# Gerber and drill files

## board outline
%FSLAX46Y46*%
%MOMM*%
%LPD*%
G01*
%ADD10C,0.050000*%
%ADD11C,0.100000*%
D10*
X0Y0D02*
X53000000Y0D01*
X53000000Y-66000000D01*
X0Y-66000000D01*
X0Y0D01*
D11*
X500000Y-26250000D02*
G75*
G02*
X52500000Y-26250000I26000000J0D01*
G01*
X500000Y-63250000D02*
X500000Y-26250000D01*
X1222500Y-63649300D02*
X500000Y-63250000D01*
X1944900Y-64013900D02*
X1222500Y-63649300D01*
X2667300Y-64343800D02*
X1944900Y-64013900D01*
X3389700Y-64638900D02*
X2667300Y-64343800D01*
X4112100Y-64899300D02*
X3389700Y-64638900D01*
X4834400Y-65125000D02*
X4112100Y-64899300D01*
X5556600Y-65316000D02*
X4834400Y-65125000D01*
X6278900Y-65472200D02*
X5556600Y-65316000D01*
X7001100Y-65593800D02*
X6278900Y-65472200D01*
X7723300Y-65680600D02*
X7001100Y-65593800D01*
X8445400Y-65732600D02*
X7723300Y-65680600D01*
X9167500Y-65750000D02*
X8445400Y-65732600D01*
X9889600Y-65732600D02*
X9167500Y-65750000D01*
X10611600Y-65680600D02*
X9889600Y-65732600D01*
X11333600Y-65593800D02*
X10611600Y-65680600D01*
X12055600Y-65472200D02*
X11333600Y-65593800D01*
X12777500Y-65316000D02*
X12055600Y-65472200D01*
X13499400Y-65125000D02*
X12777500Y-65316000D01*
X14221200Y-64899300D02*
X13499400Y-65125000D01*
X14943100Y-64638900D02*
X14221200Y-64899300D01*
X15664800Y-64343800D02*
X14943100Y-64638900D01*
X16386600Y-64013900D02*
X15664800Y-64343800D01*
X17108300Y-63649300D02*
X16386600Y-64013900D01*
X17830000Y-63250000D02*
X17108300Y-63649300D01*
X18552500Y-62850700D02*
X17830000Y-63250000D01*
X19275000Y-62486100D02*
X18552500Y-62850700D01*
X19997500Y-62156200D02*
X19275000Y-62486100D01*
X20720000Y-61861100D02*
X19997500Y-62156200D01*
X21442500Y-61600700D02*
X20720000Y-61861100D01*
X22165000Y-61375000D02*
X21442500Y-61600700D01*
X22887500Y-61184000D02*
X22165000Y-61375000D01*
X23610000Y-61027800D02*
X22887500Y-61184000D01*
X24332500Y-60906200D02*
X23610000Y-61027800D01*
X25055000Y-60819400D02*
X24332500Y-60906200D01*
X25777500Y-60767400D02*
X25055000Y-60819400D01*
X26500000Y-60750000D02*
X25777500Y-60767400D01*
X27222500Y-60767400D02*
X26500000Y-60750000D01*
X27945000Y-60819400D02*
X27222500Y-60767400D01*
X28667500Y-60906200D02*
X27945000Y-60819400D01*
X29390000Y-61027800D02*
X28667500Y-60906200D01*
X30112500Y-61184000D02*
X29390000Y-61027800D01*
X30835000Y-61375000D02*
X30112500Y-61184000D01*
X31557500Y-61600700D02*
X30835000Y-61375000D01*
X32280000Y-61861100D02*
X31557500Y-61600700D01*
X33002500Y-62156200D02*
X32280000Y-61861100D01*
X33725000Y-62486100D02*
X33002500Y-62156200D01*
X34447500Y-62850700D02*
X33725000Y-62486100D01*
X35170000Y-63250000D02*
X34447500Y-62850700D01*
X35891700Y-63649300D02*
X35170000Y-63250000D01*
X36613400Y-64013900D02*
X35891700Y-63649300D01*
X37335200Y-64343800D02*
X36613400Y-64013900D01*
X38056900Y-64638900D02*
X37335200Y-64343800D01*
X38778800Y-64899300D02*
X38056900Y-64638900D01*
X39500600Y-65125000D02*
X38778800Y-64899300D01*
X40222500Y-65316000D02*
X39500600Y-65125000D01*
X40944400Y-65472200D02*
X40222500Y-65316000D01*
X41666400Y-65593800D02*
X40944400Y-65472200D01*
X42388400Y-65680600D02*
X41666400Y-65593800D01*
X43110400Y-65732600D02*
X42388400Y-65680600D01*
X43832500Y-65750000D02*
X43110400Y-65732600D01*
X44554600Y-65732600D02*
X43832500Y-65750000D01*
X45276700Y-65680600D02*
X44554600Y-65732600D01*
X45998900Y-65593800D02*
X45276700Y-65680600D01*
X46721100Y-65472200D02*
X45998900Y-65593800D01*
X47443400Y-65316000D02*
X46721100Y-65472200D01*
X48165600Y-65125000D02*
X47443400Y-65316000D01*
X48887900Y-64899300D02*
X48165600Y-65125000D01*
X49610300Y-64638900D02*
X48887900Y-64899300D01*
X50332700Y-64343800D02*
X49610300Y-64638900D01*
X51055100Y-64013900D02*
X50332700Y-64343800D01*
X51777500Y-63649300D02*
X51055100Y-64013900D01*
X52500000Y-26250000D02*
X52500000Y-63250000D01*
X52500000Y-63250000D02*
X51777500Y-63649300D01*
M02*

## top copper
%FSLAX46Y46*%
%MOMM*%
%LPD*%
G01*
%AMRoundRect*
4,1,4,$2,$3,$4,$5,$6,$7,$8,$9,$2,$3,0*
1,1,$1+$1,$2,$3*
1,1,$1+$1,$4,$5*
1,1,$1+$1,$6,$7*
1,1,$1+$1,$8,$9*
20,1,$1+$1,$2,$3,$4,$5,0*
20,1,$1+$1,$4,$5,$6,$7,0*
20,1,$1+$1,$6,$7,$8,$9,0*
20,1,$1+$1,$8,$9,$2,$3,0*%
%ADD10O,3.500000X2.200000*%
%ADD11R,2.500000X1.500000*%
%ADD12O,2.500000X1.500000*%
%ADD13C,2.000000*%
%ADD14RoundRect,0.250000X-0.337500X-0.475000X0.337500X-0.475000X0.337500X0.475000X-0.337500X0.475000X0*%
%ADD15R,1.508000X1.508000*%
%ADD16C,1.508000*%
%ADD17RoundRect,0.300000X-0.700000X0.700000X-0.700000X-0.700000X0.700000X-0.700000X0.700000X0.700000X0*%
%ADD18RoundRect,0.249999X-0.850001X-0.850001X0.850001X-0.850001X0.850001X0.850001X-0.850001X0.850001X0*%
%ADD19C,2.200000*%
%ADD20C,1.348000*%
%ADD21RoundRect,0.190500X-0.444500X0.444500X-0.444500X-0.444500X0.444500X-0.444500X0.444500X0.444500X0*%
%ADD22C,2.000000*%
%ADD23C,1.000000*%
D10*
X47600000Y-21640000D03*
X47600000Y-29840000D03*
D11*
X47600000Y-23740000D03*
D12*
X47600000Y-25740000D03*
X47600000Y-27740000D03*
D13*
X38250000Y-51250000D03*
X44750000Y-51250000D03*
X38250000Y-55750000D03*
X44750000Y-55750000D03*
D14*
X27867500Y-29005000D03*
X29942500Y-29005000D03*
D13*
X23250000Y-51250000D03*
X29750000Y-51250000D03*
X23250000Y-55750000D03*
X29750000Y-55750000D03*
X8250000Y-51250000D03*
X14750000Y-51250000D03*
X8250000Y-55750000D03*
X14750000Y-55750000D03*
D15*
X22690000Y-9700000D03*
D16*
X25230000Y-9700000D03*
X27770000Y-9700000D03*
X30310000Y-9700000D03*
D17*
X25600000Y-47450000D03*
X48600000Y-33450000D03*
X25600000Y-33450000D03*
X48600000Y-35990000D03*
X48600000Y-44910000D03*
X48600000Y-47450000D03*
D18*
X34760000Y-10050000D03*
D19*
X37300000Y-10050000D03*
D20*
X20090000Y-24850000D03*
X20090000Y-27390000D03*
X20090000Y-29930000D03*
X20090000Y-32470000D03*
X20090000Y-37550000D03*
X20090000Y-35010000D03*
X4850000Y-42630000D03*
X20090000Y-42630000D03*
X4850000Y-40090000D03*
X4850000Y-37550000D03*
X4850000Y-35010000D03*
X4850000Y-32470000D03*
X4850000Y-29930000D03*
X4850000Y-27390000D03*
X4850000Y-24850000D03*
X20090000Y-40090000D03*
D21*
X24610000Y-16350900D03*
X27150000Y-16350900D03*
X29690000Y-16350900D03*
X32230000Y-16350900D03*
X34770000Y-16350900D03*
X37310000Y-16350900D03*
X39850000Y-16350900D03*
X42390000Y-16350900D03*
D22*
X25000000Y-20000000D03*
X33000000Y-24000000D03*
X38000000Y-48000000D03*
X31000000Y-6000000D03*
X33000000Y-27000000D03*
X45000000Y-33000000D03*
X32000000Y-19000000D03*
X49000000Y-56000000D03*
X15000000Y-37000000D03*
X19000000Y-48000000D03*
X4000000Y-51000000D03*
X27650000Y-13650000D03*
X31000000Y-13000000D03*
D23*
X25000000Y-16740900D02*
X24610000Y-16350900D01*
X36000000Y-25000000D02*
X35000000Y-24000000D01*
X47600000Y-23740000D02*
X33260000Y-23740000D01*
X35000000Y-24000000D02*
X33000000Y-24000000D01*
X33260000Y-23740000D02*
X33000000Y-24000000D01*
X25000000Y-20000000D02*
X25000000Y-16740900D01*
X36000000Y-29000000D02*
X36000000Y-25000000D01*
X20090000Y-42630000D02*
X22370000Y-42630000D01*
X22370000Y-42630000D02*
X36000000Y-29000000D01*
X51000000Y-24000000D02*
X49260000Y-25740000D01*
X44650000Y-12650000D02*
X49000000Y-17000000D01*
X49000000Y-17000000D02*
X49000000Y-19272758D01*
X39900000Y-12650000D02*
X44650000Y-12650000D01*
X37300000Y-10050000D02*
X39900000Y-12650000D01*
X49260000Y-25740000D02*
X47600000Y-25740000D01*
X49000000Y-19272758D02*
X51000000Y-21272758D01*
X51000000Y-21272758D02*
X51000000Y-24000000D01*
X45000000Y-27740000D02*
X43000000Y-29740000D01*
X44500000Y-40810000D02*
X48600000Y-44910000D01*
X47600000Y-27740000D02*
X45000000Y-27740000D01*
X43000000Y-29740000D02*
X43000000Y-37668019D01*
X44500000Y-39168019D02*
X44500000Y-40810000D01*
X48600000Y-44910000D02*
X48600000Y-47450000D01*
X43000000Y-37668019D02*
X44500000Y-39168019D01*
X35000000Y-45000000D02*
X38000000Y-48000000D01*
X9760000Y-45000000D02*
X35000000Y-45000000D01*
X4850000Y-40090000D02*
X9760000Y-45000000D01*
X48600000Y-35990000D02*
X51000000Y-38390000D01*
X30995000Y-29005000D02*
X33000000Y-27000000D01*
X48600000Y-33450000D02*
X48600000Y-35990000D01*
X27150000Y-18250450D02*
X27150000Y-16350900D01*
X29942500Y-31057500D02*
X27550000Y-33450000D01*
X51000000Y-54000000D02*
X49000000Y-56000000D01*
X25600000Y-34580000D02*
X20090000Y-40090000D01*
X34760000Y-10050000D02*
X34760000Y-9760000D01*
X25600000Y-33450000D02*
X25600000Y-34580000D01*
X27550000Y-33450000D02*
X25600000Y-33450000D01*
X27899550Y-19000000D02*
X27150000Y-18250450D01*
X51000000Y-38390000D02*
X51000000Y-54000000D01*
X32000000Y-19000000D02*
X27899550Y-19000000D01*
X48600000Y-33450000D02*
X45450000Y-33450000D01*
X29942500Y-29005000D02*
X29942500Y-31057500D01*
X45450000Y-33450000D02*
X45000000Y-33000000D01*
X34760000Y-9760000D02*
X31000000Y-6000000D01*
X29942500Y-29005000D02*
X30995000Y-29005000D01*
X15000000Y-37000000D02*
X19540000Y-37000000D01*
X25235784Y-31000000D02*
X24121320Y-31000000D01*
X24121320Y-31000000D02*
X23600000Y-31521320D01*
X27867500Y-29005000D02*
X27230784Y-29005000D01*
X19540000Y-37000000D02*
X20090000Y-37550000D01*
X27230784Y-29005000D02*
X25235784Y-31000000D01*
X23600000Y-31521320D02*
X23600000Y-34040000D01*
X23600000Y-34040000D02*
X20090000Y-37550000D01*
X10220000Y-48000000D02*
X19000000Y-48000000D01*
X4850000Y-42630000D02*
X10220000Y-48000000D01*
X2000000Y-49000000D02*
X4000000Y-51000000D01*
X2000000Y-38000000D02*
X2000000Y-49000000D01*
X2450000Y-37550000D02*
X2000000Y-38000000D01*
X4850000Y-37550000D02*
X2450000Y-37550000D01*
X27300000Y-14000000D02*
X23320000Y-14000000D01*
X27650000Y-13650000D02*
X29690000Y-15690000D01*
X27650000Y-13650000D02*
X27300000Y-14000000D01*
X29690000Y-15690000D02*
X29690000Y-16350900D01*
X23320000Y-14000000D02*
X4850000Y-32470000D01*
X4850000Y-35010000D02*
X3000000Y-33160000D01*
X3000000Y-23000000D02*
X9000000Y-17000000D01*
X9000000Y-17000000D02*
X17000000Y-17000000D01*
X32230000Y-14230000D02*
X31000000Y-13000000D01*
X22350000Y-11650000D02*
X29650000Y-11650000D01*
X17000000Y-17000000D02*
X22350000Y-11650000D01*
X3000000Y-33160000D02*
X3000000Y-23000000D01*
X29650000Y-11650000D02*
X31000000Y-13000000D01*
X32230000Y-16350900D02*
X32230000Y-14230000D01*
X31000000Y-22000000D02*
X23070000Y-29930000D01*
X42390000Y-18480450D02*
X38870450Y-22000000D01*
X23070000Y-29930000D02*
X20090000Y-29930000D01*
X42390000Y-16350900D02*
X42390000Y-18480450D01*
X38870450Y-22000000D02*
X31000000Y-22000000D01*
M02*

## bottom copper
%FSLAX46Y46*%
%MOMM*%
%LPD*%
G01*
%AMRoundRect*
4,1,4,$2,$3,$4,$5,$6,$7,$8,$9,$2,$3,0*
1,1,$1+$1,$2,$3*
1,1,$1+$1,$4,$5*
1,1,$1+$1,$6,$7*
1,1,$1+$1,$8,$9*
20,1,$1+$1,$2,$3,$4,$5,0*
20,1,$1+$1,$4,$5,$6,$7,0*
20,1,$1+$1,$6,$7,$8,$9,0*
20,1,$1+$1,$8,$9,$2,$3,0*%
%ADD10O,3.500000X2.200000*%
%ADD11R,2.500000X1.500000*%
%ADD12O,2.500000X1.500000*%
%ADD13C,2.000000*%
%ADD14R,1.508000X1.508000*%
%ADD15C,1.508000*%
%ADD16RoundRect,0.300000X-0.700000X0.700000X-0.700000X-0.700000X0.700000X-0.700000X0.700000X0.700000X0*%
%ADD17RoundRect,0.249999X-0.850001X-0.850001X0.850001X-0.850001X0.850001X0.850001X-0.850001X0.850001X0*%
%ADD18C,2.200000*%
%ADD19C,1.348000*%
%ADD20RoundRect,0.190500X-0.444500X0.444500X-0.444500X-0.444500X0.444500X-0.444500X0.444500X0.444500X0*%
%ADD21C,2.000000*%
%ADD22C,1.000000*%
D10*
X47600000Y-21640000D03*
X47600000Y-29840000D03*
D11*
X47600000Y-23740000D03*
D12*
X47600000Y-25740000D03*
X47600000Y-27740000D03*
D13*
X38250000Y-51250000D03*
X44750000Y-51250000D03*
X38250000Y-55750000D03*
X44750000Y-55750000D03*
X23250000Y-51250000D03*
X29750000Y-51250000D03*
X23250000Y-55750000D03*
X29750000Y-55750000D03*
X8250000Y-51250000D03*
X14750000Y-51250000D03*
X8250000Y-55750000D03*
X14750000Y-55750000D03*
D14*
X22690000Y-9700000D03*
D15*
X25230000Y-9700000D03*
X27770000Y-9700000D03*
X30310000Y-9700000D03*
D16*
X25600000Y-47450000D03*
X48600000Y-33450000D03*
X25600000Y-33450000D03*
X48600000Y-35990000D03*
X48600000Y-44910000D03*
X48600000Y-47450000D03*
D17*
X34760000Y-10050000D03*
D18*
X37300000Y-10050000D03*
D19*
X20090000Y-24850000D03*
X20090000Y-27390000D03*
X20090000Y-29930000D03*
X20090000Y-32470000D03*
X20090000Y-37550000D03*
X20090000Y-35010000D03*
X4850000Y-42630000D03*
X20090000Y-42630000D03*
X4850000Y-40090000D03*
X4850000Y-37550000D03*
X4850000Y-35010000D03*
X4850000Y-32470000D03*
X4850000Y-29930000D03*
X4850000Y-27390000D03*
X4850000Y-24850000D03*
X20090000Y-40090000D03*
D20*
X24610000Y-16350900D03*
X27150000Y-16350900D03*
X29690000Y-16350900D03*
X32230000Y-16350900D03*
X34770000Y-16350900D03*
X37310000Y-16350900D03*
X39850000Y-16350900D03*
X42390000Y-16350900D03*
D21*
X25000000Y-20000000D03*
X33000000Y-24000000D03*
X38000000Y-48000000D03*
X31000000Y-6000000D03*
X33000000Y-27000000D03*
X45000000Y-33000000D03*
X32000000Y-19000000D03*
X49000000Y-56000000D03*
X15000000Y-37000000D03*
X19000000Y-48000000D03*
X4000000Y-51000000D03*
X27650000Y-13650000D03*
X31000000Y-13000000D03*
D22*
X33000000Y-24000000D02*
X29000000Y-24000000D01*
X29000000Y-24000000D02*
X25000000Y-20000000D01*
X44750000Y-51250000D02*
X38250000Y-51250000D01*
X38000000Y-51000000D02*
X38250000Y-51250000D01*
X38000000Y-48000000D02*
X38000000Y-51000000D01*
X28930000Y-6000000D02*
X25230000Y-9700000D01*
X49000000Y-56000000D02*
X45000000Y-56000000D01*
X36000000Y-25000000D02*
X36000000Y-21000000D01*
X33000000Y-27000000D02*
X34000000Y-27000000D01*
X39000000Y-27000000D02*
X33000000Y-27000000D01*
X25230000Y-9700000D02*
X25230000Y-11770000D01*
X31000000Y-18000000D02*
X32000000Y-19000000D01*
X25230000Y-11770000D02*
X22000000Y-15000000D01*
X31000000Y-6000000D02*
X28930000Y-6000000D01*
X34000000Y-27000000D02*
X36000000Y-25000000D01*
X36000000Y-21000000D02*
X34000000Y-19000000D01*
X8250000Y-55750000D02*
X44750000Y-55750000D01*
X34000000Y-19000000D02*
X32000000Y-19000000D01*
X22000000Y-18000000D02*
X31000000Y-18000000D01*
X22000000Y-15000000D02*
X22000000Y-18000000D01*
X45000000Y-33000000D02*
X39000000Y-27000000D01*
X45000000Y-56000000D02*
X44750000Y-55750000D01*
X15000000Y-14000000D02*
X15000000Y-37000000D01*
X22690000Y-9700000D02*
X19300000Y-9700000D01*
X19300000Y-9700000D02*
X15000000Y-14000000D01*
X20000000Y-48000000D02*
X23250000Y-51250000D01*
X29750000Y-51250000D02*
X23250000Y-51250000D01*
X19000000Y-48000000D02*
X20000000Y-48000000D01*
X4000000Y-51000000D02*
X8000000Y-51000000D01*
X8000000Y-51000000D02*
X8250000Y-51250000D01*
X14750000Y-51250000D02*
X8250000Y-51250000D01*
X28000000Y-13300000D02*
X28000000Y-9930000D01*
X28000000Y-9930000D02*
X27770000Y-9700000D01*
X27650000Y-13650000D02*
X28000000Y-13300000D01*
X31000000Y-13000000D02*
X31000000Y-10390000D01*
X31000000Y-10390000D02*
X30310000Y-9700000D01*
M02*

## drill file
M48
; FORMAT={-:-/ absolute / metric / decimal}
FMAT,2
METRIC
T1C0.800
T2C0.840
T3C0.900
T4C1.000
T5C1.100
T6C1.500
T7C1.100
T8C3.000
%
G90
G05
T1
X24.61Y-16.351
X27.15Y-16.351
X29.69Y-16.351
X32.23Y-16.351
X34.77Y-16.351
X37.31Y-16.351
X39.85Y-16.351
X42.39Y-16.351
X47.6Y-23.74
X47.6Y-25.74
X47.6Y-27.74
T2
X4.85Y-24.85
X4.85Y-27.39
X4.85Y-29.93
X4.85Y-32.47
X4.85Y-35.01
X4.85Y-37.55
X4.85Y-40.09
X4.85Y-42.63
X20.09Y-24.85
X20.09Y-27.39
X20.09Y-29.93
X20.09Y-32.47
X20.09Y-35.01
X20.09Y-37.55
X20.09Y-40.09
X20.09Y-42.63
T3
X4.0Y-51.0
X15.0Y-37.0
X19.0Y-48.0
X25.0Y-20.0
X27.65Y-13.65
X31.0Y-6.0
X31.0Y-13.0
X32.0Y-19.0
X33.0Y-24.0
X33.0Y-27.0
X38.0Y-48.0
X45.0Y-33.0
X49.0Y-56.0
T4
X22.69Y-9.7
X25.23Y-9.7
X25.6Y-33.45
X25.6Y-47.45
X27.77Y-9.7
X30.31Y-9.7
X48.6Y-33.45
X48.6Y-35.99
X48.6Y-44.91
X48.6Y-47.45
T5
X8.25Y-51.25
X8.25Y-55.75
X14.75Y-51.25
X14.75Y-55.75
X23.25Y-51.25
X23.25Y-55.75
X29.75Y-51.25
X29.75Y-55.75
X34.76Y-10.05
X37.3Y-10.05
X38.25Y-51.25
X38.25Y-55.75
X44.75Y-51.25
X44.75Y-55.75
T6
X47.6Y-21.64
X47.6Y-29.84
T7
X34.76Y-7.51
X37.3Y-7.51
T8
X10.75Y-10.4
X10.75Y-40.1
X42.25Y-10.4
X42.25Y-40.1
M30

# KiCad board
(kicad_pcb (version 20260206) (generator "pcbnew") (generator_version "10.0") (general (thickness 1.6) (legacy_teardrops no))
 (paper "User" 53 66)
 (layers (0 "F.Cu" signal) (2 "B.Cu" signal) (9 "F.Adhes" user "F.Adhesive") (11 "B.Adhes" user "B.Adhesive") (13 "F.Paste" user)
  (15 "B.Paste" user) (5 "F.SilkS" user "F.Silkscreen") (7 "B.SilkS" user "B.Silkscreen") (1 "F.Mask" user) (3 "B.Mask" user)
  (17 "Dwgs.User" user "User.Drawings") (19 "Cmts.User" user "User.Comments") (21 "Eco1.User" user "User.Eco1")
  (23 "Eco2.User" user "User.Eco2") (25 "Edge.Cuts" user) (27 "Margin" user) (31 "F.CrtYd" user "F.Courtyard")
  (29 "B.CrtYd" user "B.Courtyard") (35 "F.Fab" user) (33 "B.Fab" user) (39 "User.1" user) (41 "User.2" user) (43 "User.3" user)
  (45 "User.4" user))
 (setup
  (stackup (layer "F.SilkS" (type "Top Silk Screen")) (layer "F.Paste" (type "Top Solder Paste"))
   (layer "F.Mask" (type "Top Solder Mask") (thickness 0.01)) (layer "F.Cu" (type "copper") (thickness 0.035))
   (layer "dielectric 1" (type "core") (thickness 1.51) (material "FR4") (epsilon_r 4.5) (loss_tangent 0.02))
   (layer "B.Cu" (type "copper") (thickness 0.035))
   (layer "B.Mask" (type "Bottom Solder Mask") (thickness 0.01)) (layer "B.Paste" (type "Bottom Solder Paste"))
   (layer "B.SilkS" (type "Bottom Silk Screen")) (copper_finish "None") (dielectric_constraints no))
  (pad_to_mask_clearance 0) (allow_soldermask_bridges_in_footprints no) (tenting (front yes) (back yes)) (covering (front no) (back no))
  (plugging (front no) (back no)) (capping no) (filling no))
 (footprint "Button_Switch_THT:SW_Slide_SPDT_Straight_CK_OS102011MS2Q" (layer "F.Cu") (at 47.6 23.74 -90)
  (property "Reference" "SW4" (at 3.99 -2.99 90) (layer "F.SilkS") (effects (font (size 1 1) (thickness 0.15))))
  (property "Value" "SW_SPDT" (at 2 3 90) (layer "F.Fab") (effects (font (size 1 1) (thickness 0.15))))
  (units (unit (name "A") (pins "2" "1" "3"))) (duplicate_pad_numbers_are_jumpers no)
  (pad "" thru_hole oval (at -2.1 0 270) (size 2.2 3.5) (drill 1.5) (layers "*.Cu" "*.Mask") (remove_unused_layers no))
  (pad "" thru_hole oval (at 6.1 0 270) (size 2.2 3.5) (drill 1.5) (layers "*.Cu" "*.Mask") (remove_unused_layers no))
  (pad "1" thru_hole rect (at 0 0 270) (size 1.5 2.5) (drill 0.8) (layers "*.Cu" "*.Mask") (remove_unused_layers no) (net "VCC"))
  (pad "2" thru_hole oval (at 2 0 270) (size 1.5 2.5) (drill 0.8) (layers "*.Cu" "*.Mask") (remove_unused_layers no) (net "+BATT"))
  (pad "3" thru_hole oval (at 4 0 270) (size 1.5 2.5) (drill 0.8) (layers "*.Cu" "*.Mask") (remove_unused_layers no) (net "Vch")))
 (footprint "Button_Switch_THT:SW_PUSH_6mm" (layer "F.Cu") (at 38.25 51.25)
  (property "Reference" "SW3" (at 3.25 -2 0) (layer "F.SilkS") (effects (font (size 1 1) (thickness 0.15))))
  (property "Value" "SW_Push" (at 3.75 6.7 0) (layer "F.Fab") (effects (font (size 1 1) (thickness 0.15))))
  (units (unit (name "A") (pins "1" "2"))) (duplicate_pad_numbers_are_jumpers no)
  (pad "1" thru_hole circle (at 0 0 90) (size 2 2) (drill 1.1) (layers "*.Cu" "*.Mask") (remove_unused_layers no) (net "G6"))
  (pad "1" thru_hole circle (at 6.5 0 90) (size 2 2) (drill 1.1) (layers "*.Cu" "*.Mask") (remove_unused_layers no) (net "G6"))
  (pad "2" thru_hole circle (at 0 4.5 90) (size 2 2) (drill 1.1) (layers "*.Cu" "*.Mask") (remove_unused_layers no) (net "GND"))
  (pad "2" thru_hole circle (at 6.5 4.5 90) (size 2 2) (drill 1.1) (layers "*.Cu" "*.Mask") (remove_unused_layers no) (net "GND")))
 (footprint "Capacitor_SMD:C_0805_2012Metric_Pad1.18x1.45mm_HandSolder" (layer "F.Cu") (at 28.905 29.005)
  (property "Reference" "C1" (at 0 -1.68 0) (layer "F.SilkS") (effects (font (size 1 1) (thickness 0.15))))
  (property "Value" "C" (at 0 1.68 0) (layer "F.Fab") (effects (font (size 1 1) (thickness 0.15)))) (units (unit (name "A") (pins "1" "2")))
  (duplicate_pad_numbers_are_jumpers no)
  (pad "1" smd roundrect (at -1.0375 0) (size 1.175 1.45) (layers "F.Cu" "F.Mask" "F.Paste") (roundrect_rratio 0.212766) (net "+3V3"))
  (pad "2" smd roundrect (at 1.0375 0) (size 1.175 1.45) (layers "F.Cu" "F.Mask" "F.Paste") (roundrect_rratio 0.212766) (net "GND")))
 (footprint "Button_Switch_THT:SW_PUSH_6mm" (layer "F.Cu") (at 23.25 51.25)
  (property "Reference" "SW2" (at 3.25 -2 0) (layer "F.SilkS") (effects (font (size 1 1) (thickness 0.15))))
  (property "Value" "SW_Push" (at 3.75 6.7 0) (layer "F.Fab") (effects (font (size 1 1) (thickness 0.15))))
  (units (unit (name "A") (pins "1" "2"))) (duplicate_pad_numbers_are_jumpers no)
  (pad "1" thru_hole circle (at 0 0 90) (size 2 2) (drill 1.1) (layers "*.Cu" "*.Mask") (remove_unused_layers no) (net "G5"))
  (pad "1" thru_hole circle (at 6.5 0 90) (size 2 2) (drill 1.1) (layers "*.Cu" "*.Mask") (remove_unused_layers no) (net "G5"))
  (pad "2" thru_hole circle (at 0 4.5 90) (size 2 2) (drill 1.1) (layers "*.Cu" "*.Mask") (remove_unused_layers no) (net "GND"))
  (pad "2" thru_hole circle (at 6.5 4.5 90) (size 2 2) (drill 1.1) (layers "*.Cu" "*.Mask") (remove_unused_layers no) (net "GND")))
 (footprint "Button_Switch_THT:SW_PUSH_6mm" (layer "F.Cu") (at 8.25 51.25)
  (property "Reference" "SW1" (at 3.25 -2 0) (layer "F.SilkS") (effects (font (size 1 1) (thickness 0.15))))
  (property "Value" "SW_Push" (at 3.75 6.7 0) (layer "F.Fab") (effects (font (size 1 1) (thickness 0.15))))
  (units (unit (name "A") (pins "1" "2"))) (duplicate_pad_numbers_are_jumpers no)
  (pad "1" thru_hole circle (at 0 0 90) (size 2 2) (drill 1.1) (layers "*.Cu" "*.Mask") (remove_unused_layers no) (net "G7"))
  (pad "1" thru_hole circle (at 6.5 0 90) (size 2 2) (drill 1.1) (layers "*.Cu" "*.Mask") (remove_unused_layers no) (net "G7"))
  (pad "2" thru_hole circle (at 0 4.5 90) (size 2 2) (drill 1.1) (layers "*.Cu" "*.Mask") (remove_unused_layers no) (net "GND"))
  (pad "2" thru_hole circle (at 6.5 4.5 90) (size 2 2) (drill 1.1) (layers "*.Cu" "*.Mask") (remove_unused_layers no) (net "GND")))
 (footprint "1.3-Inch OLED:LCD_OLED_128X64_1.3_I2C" (layer "F.Cu") (at 26.5 25.25)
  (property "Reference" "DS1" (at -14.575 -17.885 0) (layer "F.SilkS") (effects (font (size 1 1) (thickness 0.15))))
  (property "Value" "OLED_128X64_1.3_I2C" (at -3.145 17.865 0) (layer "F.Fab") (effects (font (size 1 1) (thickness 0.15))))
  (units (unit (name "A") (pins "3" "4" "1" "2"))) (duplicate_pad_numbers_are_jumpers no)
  (pad "" np_thru_hole circle (at -15.75 -14.85) (size 3 3) (drill 3) (layers "*.Cu" "*.Mask"))
  (pad "" np_thru_hole circle (at -15.75 14.85) (size 3 3) (drill 3) (layers "*.Cu" "*.Mask"))
  (pad "" np_thru_hole circle (at 15.75 -14.85) (size 3 3) (drill 3) (layers "*.Cu" "*.Mask"))
  (pad "" np_thru_hole circle (at 15.75 14.85) (size 3 3) (drill 3) (layers "*.Cu" "*.Mask"))
  (pad "1" thru_hole rect (at -3.81 -15.55) (size 1.508 1.508) (drill 1) (layers "*.Cu" "*.Mask") (remove_unused_layers no) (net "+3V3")
   (solder_mask_margin 0.102))
  (pad "2" thru_hole circle (at -1.27 -15.55) (size 1.508 1.508) (drill 1) (layers "*.Cu" "*.Mask") (remove_unused_layers no) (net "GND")
   (solder_mask_margin 0.102))
  (pad "3" thru_hole circle (at 1.27 -15.55) (size 1.508 1.508) (drill 1) (layers "*.Cu" "*.Mask") (remove_unused_layers no) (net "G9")
   (solder_mask_margin 0.102))
  (pad "4" thru_hole circle (at 3.81 -15.55) (size 1.508 1.508) (drill 1) (layers "*.Cu" "*.Mask") (remove_unused_layers no) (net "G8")
   (solder_mask_margin 0.102)))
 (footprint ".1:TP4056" (layer "B.Cu") (at 37.1 40.45 -90)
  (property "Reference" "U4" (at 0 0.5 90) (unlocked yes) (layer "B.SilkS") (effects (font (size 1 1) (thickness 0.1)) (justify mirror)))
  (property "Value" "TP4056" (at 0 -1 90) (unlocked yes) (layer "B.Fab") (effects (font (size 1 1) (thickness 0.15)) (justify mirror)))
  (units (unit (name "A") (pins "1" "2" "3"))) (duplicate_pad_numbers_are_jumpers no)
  (pad "1" thru_hole roundrect (at 7 11.5 270) (size 2 2) (drill 1) (layers "*.Cu" "*.Mask") (remove_unused_layers no)
   (roundrect_rratio 0.15) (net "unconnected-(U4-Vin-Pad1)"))
  (pad "2" thru_hole roundrect (at -7 -11.5 270) (size 2 2) (drill 1) (layers "*.Cu" "*.Mask") (remove_unused_layers no)
   (roundrect_rratio 0.15) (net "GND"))
  (pad "2" thru_hole roundrect (at -7 11.5 270) (size 2 2) (drill 1) (layers "*.Cu" "*.Mask") (remove_unused_layers no)
   (roundrect_rratio 0.15) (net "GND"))
  (pad "2" thru_hole roundrect (at -4.46 -11.5 270) (size 2 2) (drill 1) (layers "*.Cu" "*.Mask") (remove_unused_layers no)
   (roundrect_rratio 0.15) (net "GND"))
  (pad "3" thru_hole roundrect (at 4.46 -11.5 270) (size 2 2) (drill 1) (layers "*.Cu" "*.Mask") (remove_unused_layers no)
   (roundrect_rratio 0.15) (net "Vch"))
  (pad "3" thru_hole roundrect (at 7 -11.5 270) (size 2 2) (drill 1) (layers "*.Cu" "*.Mask") (remove_unused_layers no)
   (roundrect_rratio 0.15) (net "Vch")))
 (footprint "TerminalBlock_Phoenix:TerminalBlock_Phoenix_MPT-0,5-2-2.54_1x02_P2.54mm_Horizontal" (layer "B.Cu") (at 34.76 10.05)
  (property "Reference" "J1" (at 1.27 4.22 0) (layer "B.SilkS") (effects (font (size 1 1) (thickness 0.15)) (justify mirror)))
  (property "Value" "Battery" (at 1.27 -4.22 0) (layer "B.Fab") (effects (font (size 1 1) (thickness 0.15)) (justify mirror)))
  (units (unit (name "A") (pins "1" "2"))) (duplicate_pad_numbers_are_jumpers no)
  (pad "" np_thru_hole circle (at 0 -2.54) (size 1.1 1.1) (drill 1.1) (layers "*.Cu" "*.Mask"))
  (pad "" np_thru_hole circle (at 2.54 -2.54) (size 1.1 1.1) (drill 1.1) (layers "*.Cu" "*.Mask"))
  (pad "1" thru_hole roundrect (at 0 0) (size 2.2 2.2) (drill 1.1) (layers "*.Cu" "*.Mask") (remove_unused_layers no)
   (roundrect_rratio 0.113636) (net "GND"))
  (pad "2" thru_hole circle (at 2.54 0) (size 2.2 2.2) (drill 1.1) (layers "*.Cu" "*.Mask") (remove_unused_layers no) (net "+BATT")))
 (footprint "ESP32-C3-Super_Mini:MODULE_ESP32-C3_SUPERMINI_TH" (layer "B.Cu") (at 12.47 32.73)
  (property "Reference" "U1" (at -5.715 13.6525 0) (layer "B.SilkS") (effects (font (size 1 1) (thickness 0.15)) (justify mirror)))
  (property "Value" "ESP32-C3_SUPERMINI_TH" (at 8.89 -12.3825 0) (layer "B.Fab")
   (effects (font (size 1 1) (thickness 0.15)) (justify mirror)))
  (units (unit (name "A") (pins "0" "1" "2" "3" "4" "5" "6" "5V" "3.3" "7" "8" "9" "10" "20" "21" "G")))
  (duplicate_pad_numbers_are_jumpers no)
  (pad "0" thru_hole circle (at 7.62 -7.88) (size 1.348 1.348) (drill 0.84) (layers "*.Cu" "*.Mask") (remove_unused_layers no) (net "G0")
   (solder_mask_margin 0.102))
  (pad "1" thru_hole circle (at 7.62 -5.34) (size 1.348 1.348) (drill 0.84) (layers "*.Cu" "*.Mask") (remove_unused_layers no) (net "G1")
   (solder_mask_margin 0.102))
  (pad "2" thru_hole circle (at 7.62 -2.8) (size 1.348 1.348) (drill 0.84) (layers "*.Cu" "*.Mask") (remove_unused_layers no) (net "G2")
   (solder_mask_margin 0.102))
  (pad "3" thru_hole circle (at 7.62 -0.26) (size 1.348 1.348) (drill 0.84) (layers "*.Cu" "*.Mask") (remove_unused_layers no) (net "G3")
   (solder_mask_margin 0.102))
  (pad "3.3" thru_hole circle (at 7.62 4.82) (size 1.348 1.348) (drill 0.84) (layers "*.Cu" "*.Mask") (remove_unused_layers no) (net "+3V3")
   (solder_mask_margin 0.102))
  (pad "4" thru_hole circle (at 7.62 2.28) (size 1.348 1.348) (drill 0.84) (layers "*.Cu" "*.Mask") (remove_unused_layers no) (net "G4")
   (solder_mask_margin 0.102))
  (pad "5" thru_hole circle (at -7.62 9.9) (size 1.348 1.348) (drill 0.84) (layers "*.Cu" "*.Mask") (remove_unused_layers no) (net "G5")
   (solder_mask_margin 0.102))
  (pad "5V" thru_hole circle (at 7.62 9.9) (size 1.348 1.348) (drill 0.84) (layers "*.Cu" "*.Mask") (remove_unused_layers no) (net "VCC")
   (solder_mask_margin 0.102))
  (pad "6" thru_hole circle (at -7.62 7.36) (size 1.348 1.348) (drill 0.84) (layers "*.Cu" "*.Mask") (remove_unused_layers no) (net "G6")
   (solder_mask_margin 0.102))
  (pad "7" thru_hole circle (at -7.62 4.82) (size 1.348 1.348) (drill 0.84) (layers "*.Cu" "*.Mask") (remove_unused_layers no) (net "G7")
   (solder_mask_margin 0.102))
  (pad "8" thru_hole circle (at -7.62 2.28) (size 1.348 1.348) (drill 0.84) (layers "*.Cu" "*.Mask") (remove_unused_layers no) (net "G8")
   (solder_mask_margin 0.102))
  (pad "9" thru_hole circle (at -7.62 -0.26) (size 1.348 1.348) (drill 0.84) (layers "*.Cu" "*.Mask") (remove_unused_layers no) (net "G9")
   (solder_mask_margin 0.102))
  (pad "10" thru_hole circle (at -7.62 -2.8) (size 1.348 1.348) (drill 0.84) (layers "*.Cu" "*.Mask") (remove_unused_layers no) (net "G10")
   (solder_mask_margin 0.102))
  (pad "20" thru_hole circle (at -7.62 -5.34) (size 1.348 1.348) (drill 0.84) (layers "*.Cu" "*.Mask") (remove_unused_layers no) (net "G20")
   (solder_mask_margin 0.102))
  (pad "21" thru_hole circle (at -7.62 -7.88) (size 1.348 1.348) (drill 0.84) (layers "*.Cu" "*.Mask") (remove_unused_layers no) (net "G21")
   (solder_mask_margin 0.102))
  (pad "G" thru_hole circle (at 7.62 7.36) (size 1.348 1.348) (drill 0.84) (layers "*.Cu" "*.Mask") (remove_unused_layers no) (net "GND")
   (solder_mask_margin 0.102)))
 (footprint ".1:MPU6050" (layer "B.Cu") (at 33.5 22.7009 -90)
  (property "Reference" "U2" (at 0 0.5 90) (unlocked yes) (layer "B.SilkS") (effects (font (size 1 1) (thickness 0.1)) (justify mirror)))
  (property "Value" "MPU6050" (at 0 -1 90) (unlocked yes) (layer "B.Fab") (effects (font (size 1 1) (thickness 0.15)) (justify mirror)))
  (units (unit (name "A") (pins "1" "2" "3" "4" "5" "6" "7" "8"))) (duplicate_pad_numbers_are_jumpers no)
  (pad "1" thru_hole roundrect (at -6.35 8.89 270) (size 1.27 1.27) (drill 0.8) (layers "*.Cu" "*.Mask") (remove_unused_layers no)
   (roundrect_rratio 0.15) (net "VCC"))
  (pad "2" thru_hole roundrect (at -6.35 6.35 270) (size 1.27 1.27) (drill 0.8) (layers "*.Cu" "*.Mask") (remove_unused_layers no)
   (roundrect_rratio 0.15) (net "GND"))
  (pad "3" thru_hole roundrect (at -6.35 3.81 270) (size 1.27 1.27) (drill 0.8) (layers "*.Cu" "*.Mask") (remove_unused_layers no)
   (roundrect_rratio 0.15) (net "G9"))
  (pad "4" thru_hole roundrect (at -6.35 1.27 270) (size 1.27 1.27) (drill 0.8) (layers "*.Cu" "*.Mask") (remove_unused_layers no)
   (roundrect_rratio 0.15) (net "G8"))
  (pad "5" thru_hole roundrect (at -6.35 -1.27 270) (size 1.27 1.27) (drill 0.8) (layers "*.Cu" "*.Mask") (remove_unused_layers no)
   (roundrect_rratio 0.15) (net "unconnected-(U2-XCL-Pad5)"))
  (pad "6" thru_hole roundrect (at -6.35 -3.81 270) (size 1.27 1.27) (drill 0.8) (layers "*.Cu" "*.Mask") (remove_unused_layers no)
   (roundrect_rratio 0.15) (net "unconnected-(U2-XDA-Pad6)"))
  (pad "7" thru_hole roundrect (at -6.35 -6.35 270) (size 1.27 1.27) (drill 0.8) (layers "*.Cu" "*.Mask") (remove_unused_layers no)
   (roundrect_rratio 0.15) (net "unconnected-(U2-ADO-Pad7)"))
  (pad "8" thru_hole roundrect (at -6.35 -8.89 270) (size 1.27 1.27) (drill 0.8) (layers "*.Cu" "*.Mask") (remove_unused_layers no)
   (roundrect_rratio 0.15) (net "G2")))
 (gr_rect (start 0 0) (end 53 66) (stroke (width 0.05) (type solid)) (fill no) (layer "Edge.Cuts"))
 (gr_arc (start 0.5 26.25) (mid 26.5 0.25) (end 52.5 26.25) (stroke (width 0.1) (type default)) (layer "Edge.Cuts"))
 (gr_line (start 0.5 63.25) (end 0.5 26.25) (stroke (width 0.1) (type default)) (layer "Edge.Cuts"))
 (gr_line (start 1.2225 63.6493) (end 0.5 63.25) (stroke (width 0.1) (type default)) (layer "Edge.Cuts"))
 (gr_line (start 1.9449 64.0139) (end 1.2225 63.6493) (stroke (width 0.1) (type default)) (layer "Edge.Cuts"))
 (gr_line (start 2.6673 64.3438) (end 1.9449 64.0139) (stroke (width 0.1) (type default)) (layer "Edge.Cuts"))
 (gr_line (start 3.3897 64.6389) (end 2.6673 64.3438) (stroke (width 0.1) (type default)) (layer "Edge.Cuts"))
 (gr_line (start 4.1121 64.8993) (end 3.3897 64.6389) (stroke (width 0.1) (type default)) (layer "Edge.Cuts"))
 (gr_line (start 4.8344 65.125) (end 4.1121 64.8993) (stroke (width 0.1) (type default)) (layer "Edge.Cuts"))
 (gr_line (start 5.5566 65.316) (end 4.8344 65.125) (stroke (width 0.1) (type default)) (layer "Edge.Cuts"))
 (gr_line (start 6.2789 65.4722) (end 5.5566 65.316) (stroke (width 0.1) (type default)) (layer "Edge.Cuts"))
 (gr_line (start 7.0011 65.5938) (end 6.2789 65.4722) (stroke (width 0.1) (type default)) (layer "Edge.Cuts"))
 (gr_line (start 7.7233 65.6806) (end 7.0011 65.5938) (stroke (width 0.1) (type default)) (layer "Edge.Cuts"))
 (gr_line (start 8.4454 65.7326) (end 7.7233 65.6806) (stroke (width 0.1) (type default)) (layer "Edge.Cuts"))
 (gr_line (start 9.1675 65.75) (end 8.4454 65.7326) (stroke (width 0.1) (type default)) (layer "Edge.Cuts"))
 (gr_line (start 9.8896 65.7326) (end 9.1675 65.75) (stroke (width 0.1) (type default)) (layer "Edge.Cuts"))
 (gr_line (start 10.6116 65.6806) (end 9.8896 65.7326) (stroke (width 0.1) (type default)) (layer "Edge.Cuts"))
 (gr_line (start 11.3336 65.5938) (end 10.6116 65.6806) (stroke (width 0.1) (type default)) (layer "Edge.Cuts"))
 (gr_line (start 12.0556 65.4722) (end 11.3336 65.5938) (stroke (width 0.1) (type default)) (layer "Edge.Cuts"))
 (gr_line (start 12.7775 65.316) (end 12.0556 65.4722) (stroke (width 0.1) (type default)) (layer "Edge.Cuts"))
 (gr_line (start 13.4994 65.125) (end 12.7775 65.316) (stroke (width 0.1) (type default)) (layer "Edge.Cuts"))
 (gr_line (start 14.2212 64.8993) (end 13.4994 65.125) (stroke (width 0.1) (type default)) (layer "Edge.Cuts"))
 (gr_line (start 14.9431 64.6389) (end 14.2212 64.8993) (stroke (width 0.1) (type default)) (layer "Edge.Cuts"))
 (gr_line (start 15.6648 64.3438) (end 14.9431 64.6389) (stroke (width 0.1) (type default)) (layer "Edge.Cuts"))
 (gr_line (start 16.3866 64.0139) (end 15.6648 64.3438) (stroke (width 0.1) (type default)) (layer "Edge.Cuts"))
 (gr_line (start 17.1083 63.6493) (end 16.3866 64.0139) (stroke (width 0.1) (type default)) (layer "Edge.Cuts"))
 (gr_line (start 17.83 63.25) (end 17.1083 63.6493) (stroke (width 0.1) (type default)) (layer "Edge.Cuts"))
 (gr_line (start 18.5525 62.8507) (end 17.83 63.25) (stroke (width 0.1) (type default)) (layer "Edge.Cuts"))
 (gr_line (start 19.275 62.4861) (end 18.5525 62.8507) (stroke (width 0.1) (type default)) (layer "Edge.Cuts"))
 (gr_line (start 19.9975 62.1562) (end 19.275 62.4861) (stroke (width 0.1) (type default)) (layer "Edge.Cuts"))
 (gr_line (start 20.72 61.8611) (end 19.9975 62.1562) (stroke (width 0.1) (type default)) (layer "Edge.Cuts"))
 (gr_line (start 21.4425 61.6007) (end 20.72 61.8611) (stroke (width 0.1) (type default)) (layer "Edge.Cuts"))
 (gr_line (start 22.165 61.375) (end 21.4425 61.6007) (stroke (width 0.1) (type default)) (layer "Edge.Cuts"))
 (gr_line (start 22.8875 61.184) (end 22.165 61.375) (stroke (width 0.1) (type default)) (layer "Edge.Cuts"))
 (gr_line (start 23.61 61.0278) (end 22.8875 61.184) (stroke (width 0.1) (type default)) (layer "Edge.Cuts"))
 (gr_line (start 24.3325 60.9062) (end 23.61 61.0278) (stroke (width 0.1) (type default)) (layer "Edge.Cuts"))
 (gr_line (start 25.055 60.8194) (end 24.3325 60.9062) (stroke (width 0.1) (type default)) (layer "Edge.Cuts"))
 (gr_line (start 25.7775 60.7674) (end 25.055 60.8194) (stroke (width 0.1) (type default)) (layer "Edge.Cuts"))
 (gr_line (start 26.5 60.75) (end 25.7775 60.7674) (stroke (width 0.1) (type default)) (layer "Edge.Cuts"))
 (gr_line (start 27.2225 60.7674) (end 26.5 60.75) (stroke (width 0.1) (type default)) (layer "Edge.Cuts"))
 (gr_line (start 27.945 60.8194) (end 27.2225 60.7674) (stroke (width 0.1) (type default)) (layer "Edge.Cuts"))
 (gr_line (start 28.6675 60.9062) (end 27.945 60.8194) (stroke (width 0.1) (type default)) (layer "Edge.Cuts"))
 (gr_line (start 29.39 61.0278) (end 28.6675 60.9062) (stroke (width 0.1) (type default)) (layer "Edge.Cuts"))
 (gr_line (start 30.1125 61.184) (end 29.39 61.0278) (stroke (width 0.1) (type default)) (layer "Edge.Cuts"))
 (gr_line (start 30.835 61.375) (end 30.1125 61.184) (stroke (width 0.1) (type default)) (layer "Edge.Cuts"))
 (gr_line (start 31.5575 61.6007) (end 30.835 61.375) (stroke (width 0.1) (type default)) (layer "Edge.Cuts"))
 (gr_line (start 32.28 61.8611) (end 31.5575 61.6007) (stroke (width 0.1) (type default)) (layer "Edge.Cuts"))
 (gr_line (start 33.0025 62.1562) (end 32.28 61.8611) (stroke (width 0.1) (type default)) (layer "Edge.Cuts"))
 (gr_line (start 33.725 62.4861) (end 33.0025 62.1562) (stroke (width 0.1) (type default)) (layer "Edge.Cuts"))
 (gr_line (start 34.4475 62.8507) (end 33.725 62.4861) (stroke (width 0.1) (type default)) (layer "Edge.Cuts"))
 (gr_line (start 35.17 63.25) (end 34.4475 62.8507) (stroke (width 0.1) (type default)) (layer "Edge.Cuts"))
 (gr_line (start 35.8917 63.6493) (end 35.17 63.25) (stroke (width 0.1) (type default)) (layer "Edge.Cuts"))
 (gr_line (start 36.6134 64.0139) (end 35.8917 63.6493) (stroke (width 0.1) (type default)) (layer "Edge.Cuts"))
 (gr_line (start 37.3352 64.3438) (end 36.6134 64.0139) (stroke (width 0.1) (type default)) (layer "Edge.Cuts"))
 (gr_line (start 38.0569 64.6389) (end 37.3352 64.3438) (stroke (width 0.1) (type default)) (layer "Edge.Cuts"))
 (gr_line (start 38.7788 64.8993) (end 38.0569 64.6389) (stroke (width 0.1) (type default)) (layer "Edge.Cuts"))
 (gr_line (start 39.5006 65.125) (end 38.7788 64.8993) (stroke (width 0.1) (type default)) (layer "Edge.Cuts"))
 (gr_line (start 40.2225 65.316) (end 39.5006 65.125) (stroke (width 0.1) (type default)) (layer "Edge.Cuts"))
 (gr_line (start 40.9444 65.4722) (end 40.2225 65.316) (stroke (width 0.1) (type default)) (layer "Edge.Cuts"))
 (gr_line (start 41.6664 65.5938) (end 40.9444 65.4722) (stroke (width 0.1) (type default)) (layer "Edge.Cuts"))
 (gr_line (start 42.3884 65.6806) (end 41.6664 65.5938) (stroke (width 0.1) (type default)) (layer "Edge.Cuts"))
 (gr_line (start 43.1104 65.7326) (end 42.3884 65.6806) (stroke (width 0.1) (type default)) (layer "Edge.Cuts"))
 (gr_line (start 43.8325 65.75) (end 43.1104 65.7326) (stroke (width 0.1) (type default)) (layer "Edge.Cuts"))
 (gr_line (start 44.5546 65.7326) (end 43.8325 65.75) (stroke (width 0.1) (type default)) (layer "Edge.Cuts"))
 (gr_line (start 45.2767 65.6806) (end 44.5546 65.7326) (stroke (width 0.1) (type default)) (layer "Edge.Cuts"))
 (gr_line (start 45.9989 65.5938) (end 45.2767 65.6806) (stroke (width 0.1) (type default)) (layer "Edge.Cuts"))
 (gr_line (start 46.7211 65.4722) (end 45.9989 65.5938) (stroke (width 0.1) (type default)) (layer "Edge.Cuts"))
 (gr_line (start 47.4434 65.316) (end 46.7211 65.4722) (stroke (width 0.1) (type default)) (layer "Edge.Cuts"))
 (gr_line (start 48.1656 65.125) (end 47.4434 65.316) (stroke (width 0.1) (type default)) (layer "Edge.Cuts"))
 (gr_line (start 48.8879 64.8993) (end 48.1656 65.125) (stroke (width 0.1) (type default)) (layer "Edge.Cuts"))
 (gr_line (start 49.6103 64.6389) (end 48.8879 64.8993) (stroke (width 0.1) (type default)) (layer "Edge.Cuts"))
 (gr_line (start 50.3327 64.3438) (end 49.6103 64.6389) (stroke (width 0.1) (type default)) (layer "Edge.Cuts"))
 (gr_line (start 51.0551 64.0139) (end 50.3327 64.3438) (stroke (width 0.1) (type default)) (layer "Edge.Cuts"))
 (gr_line (start 51.7775 63.6493) (end 51.0551 64.0139) (stroke (width 0.1) (type default)) (layer "Edge.Cuts"))
 (gr_line (start 52.5 26.25) (end 52.5 63.25) (stroke (width 0.1) (type default)) (layer "Edge.Cuts"))
 (gr_line (start 52.5 63.25) (end 51.7775 63.6493) (stroke (width 0.1) (type default)) (layer "Edge.Cuts"))
 (segment (start 25 16.7409) (end 24.61 16.3509) (width 1) (layer "F.Cu") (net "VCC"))
 (segment (start 36 25) (end 35 24) (width 1) (layer "F.Cu") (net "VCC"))
 (segment (start 47.6 23.74) (end 33.26 23.74) (width 1) (layer "F.Cu") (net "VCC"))
 (segment (start 35 24) (end 33 24) (width 1) (layer "F.Cu") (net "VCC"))
 (segment (start 33.26 23.74) (end 33 24) (width 1) (layer "F.Cu") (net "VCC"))
 (segment (start 25 20) (end 25 16.7409) (width 1) (layer "F.Cu") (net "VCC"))
 (segment (start 36 29) (end 36 25) (width 1) (layer "F.Cu") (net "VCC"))
 (segment (start 20.09 42.63) (end 22.37 42.63) (width 1) (layer "F.Cu") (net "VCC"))
 (segment (start 22.37 42.63) (end 36 29) (width 1) (layer "F.Cu") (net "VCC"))
 (via (at 25 20) (size 2) (drill 0.9) (layers "F.Cu" "B.Cu") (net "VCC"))
 (via (at 33 24) (size 2) (drill 0.9) (layers "F.Cu" "B.Cu") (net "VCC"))
 (segment (start 33 24) (end 29 24) (width 1) (layer "B.Cu") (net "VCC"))
 (segment (start 29 24) (end 25 20) (width 1) (layer "B.Cu") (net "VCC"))
 (segment (start 51 24) (end 49.26 25.74) (width 1) (layer "F.Cu") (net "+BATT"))
 (segment (start 44.65 12.65) (end 49 17) (width 1) (layer "F.Cu") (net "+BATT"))
 (segment (start 49 17) (end 49 19.272758) (width 1) (layer "F.Cu") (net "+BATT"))
 (segment (start 39.9 12.65) (end 44.65 12.65) (width 1) (layer "F.Cu") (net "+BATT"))
 (segment (start 37.3 10.05) (end 39.9 12.65) (width 1) (layer "F.Cu") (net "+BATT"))
 (segment (start 49.26 25.74) (end 47.6 25.74) (width 1) (layer "F.Cu") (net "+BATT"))
 (segment (start 49 19.272758) (end 51 21.272758) (width 1) (layer "F.Cu") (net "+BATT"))
 (segment (start 51 21.272758) (end 51 24) (width 1) (layer "F.Cu") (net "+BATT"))
 (segment (start 45 27.74) (end 43 29.74) (width 1) (layer "F.Cu") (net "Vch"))
 (segment (start 44.5 40.81) (end 48.6 44.91) (width 1) (layer "F.Cu") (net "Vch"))
 (segment (start 47.6 27.74) (end 45 27.74) (width 1) (layer "F.Cu") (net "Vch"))
 (segment (start 43 29.74) (end 43 37.668019) (width 1) (layer "F.Cu") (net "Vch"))
 (segment (start 44.5 39.168019) (end 44.5 40.81) (width 1) (layer "F.Cu") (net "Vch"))
 (segment (start 48.6 44.91) (end 48.6 47.45) (width 1) (layer "F.Cu") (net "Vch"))
 (segment (start 43 37.668019) (end 44.5 39.168019) (width 1) (layer "F.Cu") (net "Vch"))
 (segment (start 35 45) (end 38 48) (width 1) (layer "F.Cu") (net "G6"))
 (segment (start 9.76 45) (end 35 45) (width 1) (layer "F.Cu") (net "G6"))
 (segment (start 4.85 40.09) (end 9.76 45) (width 1) (layer "F.Cu") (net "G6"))
 (via (at 38 48) (size 2) (drill 0.9) (layers "F.Cu" "B.Cu") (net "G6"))
 (segment (start 44.75 51.25) (end 38.25 51.25) (width 1) (layer "B.Cu") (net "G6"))
 (segment (start 38 51) (end 38.25 51.25) (width 1) (layer "B.Cu") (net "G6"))
 (segment (start 38 48) (end 38 51) (width 1) (layer "B.Cu") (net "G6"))
 (segment (start 48.6 35.99) (end 51 38.39) (width 1) (layer "F.Cu") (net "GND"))
 (segment (start 30.995 29.005) (end 33 27) (width 1) (layer "F.Cu") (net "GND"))
 (segment (start 48.6 33.45) (end 48.6 35.99) (width 1) (layer "F.Cu") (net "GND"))
 (segment (start 27.15 18.25045) (end 27.15 16.3509) (width 1) (layer "F.Cu") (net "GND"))
 (segment (start 29.9425 31.0575) (end 27.55 33.45) (width 1) (layer "F.Cu") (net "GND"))
 (segment (start 51 54) (end 49 56) (width 1) (layer "F.Cu") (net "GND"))
 (segment (start 25.6 34.58) (end 20.09 40.09) (width 1) (layer "F.Cu") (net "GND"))
 (segment (start 34.76 10.05) (end 34.76 9.76) (width 1) (layer "F.Cu") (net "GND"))
 (segment (start 25.6 33.45) (end 25.6 34.58) (width 1) (layer "F.Cu") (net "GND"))
 (segment (start 27.55 33.45) (end 25.6 33.45) (width 1) (layer "F.Cu") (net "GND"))
 (segment (start 27.89955 19) (end 27.15 18.25045) (width 1) (layer "F.Cu") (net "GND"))
 (segment (start 51 38.39) (end 51 54) (width 1) (layer "F.Cu") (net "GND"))
 (segment (start 32 19) (end 27.89955 19) (width 1) (layer "F.Cu") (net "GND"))
 (segment (start 48.6 33.45) (end 45.45 33.45) (width 1) (layer "F.Cu") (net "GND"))
 (segment (start 29.9425 29.005) (end 29.9425 31.0575) (width 1) (layer "F.Cu") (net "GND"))
 (segment (start 45.45 33.45) (end 45 33) (width 1) (layer "F.Cu") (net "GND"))
 (segment (start 34.76 9.76) (end 31 6) (width 1) (layer "F.Cu") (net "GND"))
 (segment (start 29.9425 29.005) (end 30.995 29.005) (width 1) (layer "F.Cu") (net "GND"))
 (via (at 31 6) (size 2) (drill 0.9) (layers "F.Cu" "B.Cu") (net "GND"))
 (via (at 33 27) (size 2) (drill 0.9) (layers "F.Cu" "B.Cu") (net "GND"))
 (via (at 45 33) (size 2) (drill 0.9) (layers "F.Cu" "B.Cu") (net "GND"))
 (via (at 32 19) (size 2) (drill 0.9) (layers "F.Cu" "B.Cu") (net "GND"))
 (via (at 49 56) (size 2) (drill 0.9) (layers "F.Cu" "B.Cu") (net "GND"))
 (segment (start 28.93 6) (end 25.23 9.7) (width 1) (layer "B.Cu") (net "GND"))
 (segment (start 49 56) (end 45 56) (width 1) (layer "B.Cu") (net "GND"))
 (segment (start 36 25) (end 36 21) (width 1) (layer "B.Cu") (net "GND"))
 (segment (start 33 27) (end 34 27) (width 1) (layer "B.Cu") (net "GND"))
 (segment (start 39 27) (end 33 27) (width 1) (layer "B.Cu") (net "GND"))
 (segment (start 25.23 9.7) (end 25.23 11.77) (width 1) (layer "B.Cu") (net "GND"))
 (segment (start 31 18) (end 32 19) (width 1) (layer "B.Cu") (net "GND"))
 (segment (start 25.23 11.77) (end 22 15) (width 1) (layer "B.Cu") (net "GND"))
 (segment (start 31 6) (end 28.93 6) (width 1) (layer "B.Cu") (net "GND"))
 (segment (start 34 27) (end 36 25) (width 1) (layer "B.Cu") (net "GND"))
 (segment (start 36 21) (end 34 19) (width 1) (layer "B.Cu") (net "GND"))
 (segment (start 8.25 55.75) (end 44.75 55.75) (width 1) (layer "B.Cu") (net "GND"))
 (segment (start 34 19) (end 32 19) (width 1) (layer "B.Cu") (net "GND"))
 (segment (start 22 18) (end 31 18) (width 1) (layer "B.Cu") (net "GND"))
 (segment (start 22 15) (end 22 18) (width 1) (layer "B.Cu") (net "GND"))
 (segment (start 45 33) (end 39 27) (width 1) (layer "B.Cu") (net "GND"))
 (segment (start 45 56) (end 44.75 55.75) (width 1) (layer "B.Cu") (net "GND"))
 (segment (start 15 37) (end 19.54 37) (width 1) (layer "F.Cu") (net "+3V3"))
 (segment (start 25.235784 31) (end 24.12132 31) (width 1) (layer "F.Cu") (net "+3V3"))
 (segment (start 24.12132 31) (end 23.6 31.52132) (width 1) (layer "F.Cu") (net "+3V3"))
 (segment (start 27.8675 29.005) (end 27.230784 29.005) (width 1) (layer "F.Cu") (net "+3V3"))
 (segment (start 19.54 37) (end 20.09 37.55) (width 1) (layer "F.Cu") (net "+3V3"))
 (segment (start 27.230784 29.005) (end 25.235784 31) (width 1) (layer "F.Cu") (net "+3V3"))
 (segment (start 23.6 31.52132) (end 23.6 34.04) (width 1) (layer "F.Cu") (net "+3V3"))
 (segment (start 23.6 34.04) (end 20.09 37.55) (width 1) (layer "F.Cu") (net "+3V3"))
 (via (at 15 37) (size 2) (drill 0.9) (layers "F.Cu" "B.Cu") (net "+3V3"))
 (segment (start 15 14) (end 15 37) (width 1) (layer "B.Cu") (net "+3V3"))
 (segment (start 22.69 9.7) (end 19.3 9.7) (width 1) (layer "B.Cu") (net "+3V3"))
 (segment (start 19.3 9.7) (end 15 14) (width 1) (layer "B.Cu") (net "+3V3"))
 (segment (start 10.22 48) (end 19 48) (width 1) (layer "F.Cu") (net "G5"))
 (segment (start 4.85 42.63) (end 10.22 48) (width 1) (layer "F.Cu") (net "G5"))
 (via (at 19 48) (size 2) (drill 0.9) (layers "F.Cu" "B.Cu") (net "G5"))
 (segment (start 20 48) (end 23.25 51.25) (width 1) (layer "B.Cu") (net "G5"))
 (segment (start 29.75 51.25) (end 23.25 51.25) (width 1) (layer "B.Cu") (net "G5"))
 (segment (start 19 48) (end 20 48) (width 1) (layer "B.Cu") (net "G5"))
 (segment (start 2 49) (end 4 51) (width 1) (layer "F.Cu") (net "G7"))
 (segment (start 2 38) (end 2 49) (width 1) (layer "F.Cu") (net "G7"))
 (segment (start 2.45 37.55) (end 2 38) (width 1) (layer "F.Cu") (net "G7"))
 (segment (start 4.85 37.55) (end 2.45 37.55) (width 1) (layer "F.Cu") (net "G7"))
 (via (at 4 51) (size 2) (drill 0.9) (layers "F.Cu" "B.Cu") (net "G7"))
 (segment (start 4 51) (end 8 51) (width 1) (layer "B.Cu") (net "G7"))
 (segment (start 8 51) (end 8.25 51.25) (width 1) (layer "B.Cu") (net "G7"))
 (segment (start 14.75 51.25) (end 8.25 51.25) (width 1) (layer "B.Cu") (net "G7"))
 (segment (start 27.3 14) (end 23.32 14) (width 1) (layer "F.Cu") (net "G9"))
 (segment (start 27.65 13.65) (end 29.69 15.69) (width 1) (layer "F.Cu") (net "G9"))
 (segment (start 27.65 13.65) (end 27.3 14) (width 1) (layer "F.Cu") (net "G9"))
 (segment (start 29.69 15.69) (end 29.69 16.3509) (width 1) (layer "F.Cu") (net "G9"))
 (segment (start 23.32 14) (end 4.85 32.47) (width 1) (layer "F.Cu") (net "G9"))
 (via (at 27.65 13.65) (size 2) (drill 0.9) (layers "F.Cu" "B.Cu") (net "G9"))
 (segment (start 28 13.3) (end 28 9.93) (width 1) (layer "B.Cu") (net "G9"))
 (segment (start 28 9.93) (end 27.77 9.7) (width 1) (layer "B.Cu") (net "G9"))
 (segment (start 27.65 13.65) (end 28 13.3) (width 1) (layer "B.Cu") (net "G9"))
 (segment (start 4.85 35.01) (end 3 33.16) (width 1) (layer "F.Cu") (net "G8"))
 (segment (start 3 23) (end 9 17) (width 1) (layer "F.Cu") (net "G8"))
 (segment (start 9 17) (end 17 17) (width 1) (layer "F.Cu") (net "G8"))
 (segment (start 32.23 14.23) (end 31 13) (width 1) (layer "F.Cu") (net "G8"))
 (segment (start 22.35 11.65) (end 29.65 11.65) (width 1) (layer "F.Cu") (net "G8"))
 (segment (start 17 17) (end 22.35 11.65) (width 1) (layer "F.Cu") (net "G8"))
 (segment (start 3 33.16) (end 3 23) (width 1) (layer "F.Cu") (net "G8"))
 (segment (start 29.65 11.65) (end 31 13) (width 1) (layer "F.Cu") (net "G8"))
 (segment (start 32.23 16.3509) (end 32.23 14.23) (width 1) (layer "F.Cu") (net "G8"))
 (via (at 31 13) (size 2) (drill 0.9) (layers "F.Cu" "B.Cu") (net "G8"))
 (segment (start 31 13) (end 31 10.39) (width 1) (layer "B.Cu") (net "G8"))
 (segment (start 31 10.39) (end 30.31 9.7) (width 1) (layer "B.Cu") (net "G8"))
 (segment (start 31 22) (end 23.07 29.93) (width 1) (layer "F.Cu") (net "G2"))
 (segment (start 42.39 18.48045) (end 38.87045 22) (width 1) (layer "F.Cu") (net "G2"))
 (segment (start 23.07 29.93) (end 20.09 29.93) (width 1) (layer "F.Cu") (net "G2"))
 (segment (start 42.39 16.3509) (end 42.39 18.48045) (width 1) (layer "F.Cu") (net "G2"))
 (segment (start 38.87045 22) (end 31 22) (width 1) (layer "F.Cu") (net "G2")))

